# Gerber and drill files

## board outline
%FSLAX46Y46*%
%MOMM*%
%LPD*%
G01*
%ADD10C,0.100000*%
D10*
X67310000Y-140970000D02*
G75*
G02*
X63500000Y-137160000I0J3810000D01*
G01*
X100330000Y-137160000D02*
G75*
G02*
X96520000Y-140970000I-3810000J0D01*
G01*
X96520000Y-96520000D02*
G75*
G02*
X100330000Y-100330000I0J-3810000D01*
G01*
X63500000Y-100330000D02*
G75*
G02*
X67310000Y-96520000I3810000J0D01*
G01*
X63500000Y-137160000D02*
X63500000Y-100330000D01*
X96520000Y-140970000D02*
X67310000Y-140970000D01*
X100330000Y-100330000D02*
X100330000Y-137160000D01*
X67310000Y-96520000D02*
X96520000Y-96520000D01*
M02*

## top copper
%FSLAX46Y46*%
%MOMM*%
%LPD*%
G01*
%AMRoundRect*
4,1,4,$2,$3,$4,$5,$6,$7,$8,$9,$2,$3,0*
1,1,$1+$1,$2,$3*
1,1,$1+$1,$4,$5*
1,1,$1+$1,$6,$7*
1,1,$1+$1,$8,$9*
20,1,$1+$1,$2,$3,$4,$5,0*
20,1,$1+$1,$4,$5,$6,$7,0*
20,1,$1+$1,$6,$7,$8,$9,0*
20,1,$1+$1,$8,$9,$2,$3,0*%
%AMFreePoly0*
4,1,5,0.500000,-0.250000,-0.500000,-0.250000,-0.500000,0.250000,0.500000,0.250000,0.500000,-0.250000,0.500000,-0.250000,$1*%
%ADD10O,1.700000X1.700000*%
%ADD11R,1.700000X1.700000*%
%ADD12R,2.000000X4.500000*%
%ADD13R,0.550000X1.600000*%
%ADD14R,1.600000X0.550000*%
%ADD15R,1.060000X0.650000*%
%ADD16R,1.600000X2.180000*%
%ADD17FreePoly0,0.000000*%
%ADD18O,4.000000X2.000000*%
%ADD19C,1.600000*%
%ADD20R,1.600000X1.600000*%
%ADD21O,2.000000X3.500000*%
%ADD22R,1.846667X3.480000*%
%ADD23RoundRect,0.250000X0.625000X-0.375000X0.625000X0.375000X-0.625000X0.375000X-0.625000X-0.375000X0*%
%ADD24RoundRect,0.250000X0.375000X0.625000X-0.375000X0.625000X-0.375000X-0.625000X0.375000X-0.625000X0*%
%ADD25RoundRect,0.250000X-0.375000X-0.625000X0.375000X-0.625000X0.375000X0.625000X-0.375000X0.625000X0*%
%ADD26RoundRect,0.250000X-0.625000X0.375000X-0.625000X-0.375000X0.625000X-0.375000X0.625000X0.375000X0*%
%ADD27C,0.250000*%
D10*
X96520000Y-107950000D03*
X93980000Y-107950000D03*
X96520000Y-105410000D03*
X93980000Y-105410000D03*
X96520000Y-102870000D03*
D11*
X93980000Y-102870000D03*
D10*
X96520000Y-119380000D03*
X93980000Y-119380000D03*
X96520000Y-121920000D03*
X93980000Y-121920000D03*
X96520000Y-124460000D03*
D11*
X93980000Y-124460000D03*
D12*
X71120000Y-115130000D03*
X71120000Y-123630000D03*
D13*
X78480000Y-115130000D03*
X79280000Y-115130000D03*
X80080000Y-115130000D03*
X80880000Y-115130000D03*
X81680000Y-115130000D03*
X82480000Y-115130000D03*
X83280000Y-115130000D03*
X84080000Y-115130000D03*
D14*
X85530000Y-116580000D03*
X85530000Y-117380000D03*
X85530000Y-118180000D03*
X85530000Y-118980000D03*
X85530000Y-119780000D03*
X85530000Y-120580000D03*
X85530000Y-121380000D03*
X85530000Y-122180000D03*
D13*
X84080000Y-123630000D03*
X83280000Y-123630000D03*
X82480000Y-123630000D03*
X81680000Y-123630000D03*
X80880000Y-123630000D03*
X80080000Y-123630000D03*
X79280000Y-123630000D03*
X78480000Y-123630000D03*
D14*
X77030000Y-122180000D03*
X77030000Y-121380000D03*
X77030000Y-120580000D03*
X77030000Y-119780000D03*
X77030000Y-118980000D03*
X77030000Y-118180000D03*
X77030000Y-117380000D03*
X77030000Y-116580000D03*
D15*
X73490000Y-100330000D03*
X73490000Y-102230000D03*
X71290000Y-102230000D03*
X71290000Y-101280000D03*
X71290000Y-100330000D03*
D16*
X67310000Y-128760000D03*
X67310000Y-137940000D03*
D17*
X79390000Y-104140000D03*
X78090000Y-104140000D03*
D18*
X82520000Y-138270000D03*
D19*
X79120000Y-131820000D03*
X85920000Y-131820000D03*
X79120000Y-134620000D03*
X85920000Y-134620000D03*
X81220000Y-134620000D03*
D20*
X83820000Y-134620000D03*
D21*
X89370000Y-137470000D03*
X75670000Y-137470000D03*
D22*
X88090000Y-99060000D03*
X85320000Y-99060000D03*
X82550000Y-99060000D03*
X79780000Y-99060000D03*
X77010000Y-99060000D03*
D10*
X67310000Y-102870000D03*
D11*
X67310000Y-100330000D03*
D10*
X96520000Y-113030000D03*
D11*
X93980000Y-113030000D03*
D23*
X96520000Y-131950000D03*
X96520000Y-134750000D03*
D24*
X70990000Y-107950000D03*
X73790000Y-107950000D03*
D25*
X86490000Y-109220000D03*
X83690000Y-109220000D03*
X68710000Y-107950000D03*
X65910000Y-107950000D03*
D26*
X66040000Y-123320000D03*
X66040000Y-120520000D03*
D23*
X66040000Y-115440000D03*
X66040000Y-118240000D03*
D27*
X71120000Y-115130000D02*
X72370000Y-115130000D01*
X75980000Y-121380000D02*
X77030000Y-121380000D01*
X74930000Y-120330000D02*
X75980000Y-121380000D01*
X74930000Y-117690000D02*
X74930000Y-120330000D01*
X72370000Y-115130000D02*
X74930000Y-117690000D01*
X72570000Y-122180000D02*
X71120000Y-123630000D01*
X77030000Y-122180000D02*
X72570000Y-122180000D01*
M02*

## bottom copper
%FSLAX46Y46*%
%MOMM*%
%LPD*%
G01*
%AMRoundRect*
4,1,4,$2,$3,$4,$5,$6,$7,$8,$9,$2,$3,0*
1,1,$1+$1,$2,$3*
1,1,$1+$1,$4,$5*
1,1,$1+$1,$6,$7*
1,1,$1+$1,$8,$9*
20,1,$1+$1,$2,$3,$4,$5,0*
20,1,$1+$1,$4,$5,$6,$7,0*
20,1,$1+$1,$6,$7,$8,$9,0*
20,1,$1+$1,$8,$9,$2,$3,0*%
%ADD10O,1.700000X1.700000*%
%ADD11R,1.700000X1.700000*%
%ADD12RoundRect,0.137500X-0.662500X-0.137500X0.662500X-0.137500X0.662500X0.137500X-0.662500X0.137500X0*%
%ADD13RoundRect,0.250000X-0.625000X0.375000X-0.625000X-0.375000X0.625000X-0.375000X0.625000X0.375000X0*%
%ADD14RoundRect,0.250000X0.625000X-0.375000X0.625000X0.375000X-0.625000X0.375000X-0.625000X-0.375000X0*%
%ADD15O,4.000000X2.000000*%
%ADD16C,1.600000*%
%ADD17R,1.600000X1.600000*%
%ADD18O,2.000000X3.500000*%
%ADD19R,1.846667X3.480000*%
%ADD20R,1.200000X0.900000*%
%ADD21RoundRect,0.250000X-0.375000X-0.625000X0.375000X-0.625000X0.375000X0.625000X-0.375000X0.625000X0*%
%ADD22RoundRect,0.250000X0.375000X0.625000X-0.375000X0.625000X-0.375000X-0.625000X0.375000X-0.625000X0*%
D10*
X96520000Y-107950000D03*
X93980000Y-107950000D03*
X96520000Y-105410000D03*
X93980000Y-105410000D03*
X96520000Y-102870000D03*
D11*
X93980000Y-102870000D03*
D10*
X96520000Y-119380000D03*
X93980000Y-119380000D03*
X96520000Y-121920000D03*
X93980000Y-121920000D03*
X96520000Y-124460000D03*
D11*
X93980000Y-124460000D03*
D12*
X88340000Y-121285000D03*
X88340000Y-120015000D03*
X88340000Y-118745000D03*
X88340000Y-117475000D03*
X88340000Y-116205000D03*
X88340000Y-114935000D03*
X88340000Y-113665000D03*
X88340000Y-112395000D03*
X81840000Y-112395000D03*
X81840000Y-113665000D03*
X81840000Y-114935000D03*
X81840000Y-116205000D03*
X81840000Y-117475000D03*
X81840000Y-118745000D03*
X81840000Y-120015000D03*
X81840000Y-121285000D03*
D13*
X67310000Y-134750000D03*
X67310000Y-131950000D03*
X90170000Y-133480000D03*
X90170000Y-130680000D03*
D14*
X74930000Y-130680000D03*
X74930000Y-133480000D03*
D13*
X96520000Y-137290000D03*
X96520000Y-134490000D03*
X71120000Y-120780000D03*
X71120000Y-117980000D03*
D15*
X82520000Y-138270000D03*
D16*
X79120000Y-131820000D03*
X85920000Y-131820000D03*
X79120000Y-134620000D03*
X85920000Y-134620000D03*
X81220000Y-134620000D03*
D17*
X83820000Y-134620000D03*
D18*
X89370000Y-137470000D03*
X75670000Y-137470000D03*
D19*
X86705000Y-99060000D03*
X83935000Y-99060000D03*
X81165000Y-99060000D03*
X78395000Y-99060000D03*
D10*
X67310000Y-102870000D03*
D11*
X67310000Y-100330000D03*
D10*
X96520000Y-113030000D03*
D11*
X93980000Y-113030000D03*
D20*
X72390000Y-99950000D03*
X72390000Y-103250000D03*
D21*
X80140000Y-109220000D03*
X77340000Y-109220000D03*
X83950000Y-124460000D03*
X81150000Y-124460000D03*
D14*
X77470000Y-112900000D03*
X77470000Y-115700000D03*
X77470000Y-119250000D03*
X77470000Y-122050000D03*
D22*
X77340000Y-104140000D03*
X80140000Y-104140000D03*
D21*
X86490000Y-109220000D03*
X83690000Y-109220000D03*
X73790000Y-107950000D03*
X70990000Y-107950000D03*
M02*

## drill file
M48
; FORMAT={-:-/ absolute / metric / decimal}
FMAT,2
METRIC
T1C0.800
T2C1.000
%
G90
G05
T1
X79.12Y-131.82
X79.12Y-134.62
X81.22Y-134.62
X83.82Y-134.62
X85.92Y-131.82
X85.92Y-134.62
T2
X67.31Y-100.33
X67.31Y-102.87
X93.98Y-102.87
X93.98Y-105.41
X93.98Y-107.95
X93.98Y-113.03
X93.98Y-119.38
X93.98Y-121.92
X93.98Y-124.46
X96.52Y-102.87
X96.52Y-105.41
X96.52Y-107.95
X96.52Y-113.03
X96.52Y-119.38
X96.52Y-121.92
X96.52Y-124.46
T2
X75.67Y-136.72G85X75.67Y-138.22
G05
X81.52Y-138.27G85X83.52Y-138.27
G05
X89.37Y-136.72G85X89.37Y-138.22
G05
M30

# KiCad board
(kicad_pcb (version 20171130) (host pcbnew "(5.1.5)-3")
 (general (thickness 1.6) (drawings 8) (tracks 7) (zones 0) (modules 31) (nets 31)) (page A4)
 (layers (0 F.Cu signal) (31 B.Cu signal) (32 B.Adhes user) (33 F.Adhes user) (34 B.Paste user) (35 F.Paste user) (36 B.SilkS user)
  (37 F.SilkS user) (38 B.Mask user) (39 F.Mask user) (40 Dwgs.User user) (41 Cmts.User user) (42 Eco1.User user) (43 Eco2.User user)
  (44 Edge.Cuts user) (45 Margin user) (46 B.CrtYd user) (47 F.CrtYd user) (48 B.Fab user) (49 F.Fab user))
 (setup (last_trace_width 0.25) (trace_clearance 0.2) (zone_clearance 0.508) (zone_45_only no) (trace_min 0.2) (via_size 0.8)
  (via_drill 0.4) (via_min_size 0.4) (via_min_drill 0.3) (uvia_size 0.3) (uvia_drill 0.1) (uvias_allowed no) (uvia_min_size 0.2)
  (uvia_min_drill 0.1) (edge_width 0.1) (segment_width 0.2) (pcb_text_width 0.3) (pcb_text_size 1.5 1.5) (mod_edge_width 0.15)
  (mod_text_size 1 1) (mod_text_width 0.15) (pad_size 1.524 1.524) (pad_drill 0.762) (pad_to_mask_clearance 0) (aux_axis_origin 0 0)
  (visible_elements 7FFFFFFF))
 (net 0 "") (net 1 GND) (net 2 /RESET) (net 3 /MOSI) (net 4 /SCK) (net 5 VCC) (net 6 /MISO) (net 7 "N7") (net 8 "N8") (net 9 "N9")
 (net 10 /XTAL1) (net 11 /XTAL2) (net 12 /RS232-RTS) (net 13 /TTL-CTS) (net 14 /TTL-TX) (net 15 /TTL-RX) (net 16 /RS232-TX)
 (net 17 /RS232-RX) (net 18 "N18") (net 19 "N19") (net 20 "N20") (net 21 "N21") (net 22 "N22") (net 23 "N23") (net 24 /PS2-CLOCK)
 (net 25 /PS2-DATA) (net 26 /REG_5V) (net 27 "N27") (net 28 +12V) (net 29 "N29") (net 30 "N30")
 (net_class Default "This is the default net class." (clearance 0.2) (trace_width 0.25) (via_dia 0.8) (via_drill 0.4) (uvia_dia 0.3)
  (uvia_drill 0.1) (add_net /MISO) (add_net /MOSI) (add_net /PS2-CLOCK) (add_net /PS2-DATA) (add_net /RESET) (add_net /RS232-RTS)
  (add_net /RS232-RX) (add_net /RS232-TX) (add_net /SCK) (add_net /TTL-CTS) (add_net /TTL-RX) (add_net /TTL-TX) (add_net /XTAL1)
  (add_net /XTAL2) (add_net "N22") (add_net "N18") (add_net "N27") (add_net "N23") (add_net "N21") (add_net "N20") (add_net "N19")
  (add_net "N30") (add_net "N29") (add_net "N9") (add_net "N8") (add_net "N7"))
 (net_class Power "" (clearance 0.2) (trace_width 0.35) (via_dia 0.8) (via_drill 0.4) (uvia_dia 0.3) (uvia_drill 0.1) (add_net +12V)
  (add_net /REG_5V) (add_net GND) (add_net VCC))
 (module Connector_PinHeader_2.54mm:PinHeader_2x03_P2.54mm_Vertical (layer F.Cu) (at 93.98 102.87)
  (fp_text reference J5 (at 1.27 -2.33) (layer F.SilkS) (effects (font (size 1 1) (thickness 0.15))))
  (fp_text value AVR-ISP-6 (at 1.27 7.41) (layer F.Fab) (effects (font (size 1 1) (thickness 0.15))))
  (pad 6 thru_hole oval (at 2.54 5.08) (size 1.7 1.7) (drill 1) (layers *.Cu *.Mask) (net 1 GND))
  (pad 5 thru_hole oval (at 0 5.08) (size 1.7 1.7) (drill 1) (layers *.Cu *.Mask) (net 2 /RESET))
  (pad 4 thru_hole oval (at 2.54 2.54) (size 1.7 1.7) (drill 1) (layers *.Cu *.Mask) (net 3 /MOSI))
  (pad 3 thru_hole oval (at 0 2.54) (size 1.7 1.7) (drill 1) (layers *.Cu *.Mask) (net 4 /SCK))
  (pad 2 thru_hole oval (at 2.54 0) (size 1.7 1.7) (drill 1) (layers *.Cu *.Mask) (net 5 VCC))
  (pad 1 thru_hole rect (at 0 0) (size 1.7 1.7) (drill 1) (layers *.Cu *.Mask) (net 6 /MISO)))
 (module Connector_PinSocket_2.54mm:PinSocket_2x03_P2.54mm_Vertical (layer F.Cu) (at 93.98 124.46 180)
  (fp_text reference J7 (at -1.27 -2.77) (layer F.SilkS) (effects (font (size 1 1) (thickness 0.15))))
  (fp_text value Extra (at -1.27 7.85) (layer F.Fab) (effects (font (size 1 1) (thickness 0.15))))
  (pad 6 thru_hole oval (at -2.54 5.08 180) (size 1.7 1.7) (drill 1) (layers *.Cu *.Mask) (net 1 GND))
  (pad 5 thru_hole oval (at 0 5.08 180) (size 1.7 1.7) (drill 1) (layers *.Cu *.Mask) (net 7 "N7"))
  (pad 4 thru_hole oval (at -2.54 2.54 180) (size 1.7 1.7) (drill 1) (layers *.Cu *.Mask) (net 1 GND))
  (pad 3 thru_hole oval (at 0 2.54 180) (size 1.7 1.7) (drill 1) (layers *.Cu *.Mask) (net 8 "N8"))
  (pad 2 thru_hole oval (at -2.54 0 180) (size 1.7 1.7) (drill 1) (layers *.Cu *.Mask) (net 1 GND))
  (pad 1 thru_hole rect (at 0 0 180) (size 1.7 1.7) (drill 1) (layers *.Cu *.Mask) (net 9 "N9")))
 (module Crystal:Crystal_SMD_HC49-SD (layer F.Cu) (at 71.12 119.38 90)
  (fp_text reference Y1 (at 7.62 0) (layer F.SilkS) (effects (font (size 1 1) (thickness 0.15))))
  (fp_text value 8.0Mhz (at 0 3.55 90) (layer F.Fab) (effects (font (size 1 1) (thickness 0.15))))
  (pad 2 smd rect (at 4.25 0 90) (size 4.5 2) (layers F.Cu F.Paste F.Mask) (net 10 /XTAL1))
  (pad 1 smd rect (at -4.25 0 90) (size 4.5 2) (layers F.Cu F.Paste F.Mask) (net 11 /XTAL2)))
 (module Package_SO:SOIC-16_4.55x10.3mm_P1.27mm (layer B.Cu) (at 85.09 116.84)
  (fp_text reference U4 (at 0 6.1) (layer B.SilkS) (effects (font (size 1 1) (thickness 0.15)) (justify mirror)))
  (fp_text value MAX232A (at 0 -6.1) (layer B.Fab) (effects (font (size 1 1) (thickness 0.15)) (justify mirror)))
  (pad 16 smd roundrect (at 3.25 4.445) (size 1.6 0.55) (layers B.Cu B.Paste B.Mask) (roundrect_rratio 0.25) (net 5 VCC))
  (pad 15 smd roundrect (at 3.25 3.175) (size 1.6 0.55) (layers B.Cu B.Paste B.Mask) (roundrect_rratio 0.25) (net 1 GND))
  (pad 14 smd roundrect (at 3.25 1.905) (size 1.6 0.55) (layers B.Cu B.Paste B.Mask) (roundrect_rratio 0.25))
  (pad 13 smd roundrect (at 3.25 0.635) (size 1.6 0.55) (layers B.Cu B.Paste B.Mask) (roundrect_rratio 0.25) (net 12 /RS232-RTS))
  (pad 12 smd roundrect (at 3.25 -0.635) (size 1.6 0.55) (layers B.Cu B.Paste B.Mask) (roundrect_rratio 0.25) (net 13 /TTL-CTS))
  (pad 11 smd roundrect (at 3.25 -1.905) (size 1.6 0.55) (layers B.Cu B.Paste B.Mask) (roundrect_rratio 0.25) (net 1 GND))
  (pad 10 smd roundrect (at 3.25 -3.175) (size 1.6 0.55) (layers B.Cu B.Paste B.Mask) (roundrect_rratio 0.25) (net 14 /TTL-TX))
  (pad 9 smd roundrect (at 3.25 -4.445) (size 1.6 0.55) (layers B.Cu B.Paste B.Mask) (roundrect_rratio 0.25) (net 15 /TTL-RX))
  (pad 8 smd roundrect (at -3.25 -4.445) (size 1.6 0.55) (layers B.Cu B.Paste B.Mask) (roundrect_rratio 0.25) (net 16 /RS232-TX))
  (pad 7 smd roundrect (at -3.25 -3.175) (size 1.6 0.55) (layers B.Cu B.Paste B.Mask) (roundrect_rratio 0.25) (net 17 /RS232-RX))
  (pad 6 smd roundrect (at -3.25 -1.905) (size 1.6 0.55) (layers B.Cu B.Paste B.Mask) (roundrect_rratio 0.25) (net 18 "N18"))
  (pad 5 smd roundrect (at -3.25 -0.635) (size 1.6 0.55) (layers B.Cu B.Paste B.Mask) (roundrect_rratio 0.25) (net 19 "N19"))
  (pad 4 smd roundrect (at -3.25 0.635) (size 1.6 0.55) (layers B.Cu B.Paste B.Mask) (roundrect_rratio 0.25) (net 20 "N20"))
  (pad 3 smd roundrect (at -3.25 1.905) (size 1.6 0.55) (layers B.Cu B.Paste B.Mask) (roundrect_rratio 0.25) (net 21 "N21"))
  (pad 2 smd roundrect (at -3.25 3.175) (size 1.6 0.55) (layers B.Cu B.Paste B.Mask) (roundrect_rratio 0.25) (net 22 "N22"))
  (pad 1 smd roundrect (at -3.25 4.445) (size 1.6 0.55) (layers B.Cu B.Paste B.Mask) (roundrect_rratio 0.25) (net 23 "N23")))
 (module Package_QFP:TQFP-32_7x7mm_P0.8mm (layer F.Cu) (at 81.28 119.38)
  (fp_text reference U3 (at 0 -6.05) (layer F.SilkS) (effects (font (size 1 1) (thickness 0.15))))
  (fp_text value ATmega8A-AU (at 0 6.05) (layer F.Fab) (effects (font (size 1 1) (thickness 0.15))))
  (pad 32 smd rect (at -2.8 -4.25 90) (size 1.6 0.55) (layers F.Cu F.Paste F.Mask) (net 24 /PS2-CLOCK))
  (pad 31 smd rect (at -2 -4.25 90) (size 1.6 0.55) (layers F.Cu F.Paste F.Mask) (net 14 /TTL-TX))
  (pad 30 smd rect (at -1.2 -4.25 90) (size 1.6 0.55) (layers F.Cu F.Paste F.Mask) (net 15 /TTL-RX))
  (pad 29 smd rect (at -0.4 -4.25 90) (size 1.6 0.55) (layers F.Cu F.Paste F.Mask) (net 2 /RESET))
  (pad 28 smd rect (at 0.4 -4.25 90) (size 1.6 0.55) (layers F.Cu F.Paste F.Mask))
  (pad 27 smd rect (at 1.2 -4.25 90) (size 1.6 0.55) (layers F.Cu F.Paste F.Mask))
  (pad 26 smd rect (at 2 -4.25 90) (size 1.6 0.55) (layers F.Cu F.Paste F.Mask))
  (pad 25 smd rect (at 2.8 -4.25 90) (size 1.6 0.55) (layers F.Cu F.Paste F.Mask) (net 7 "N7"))
  (pad 24 smd rect (at 4.25 -2.8) (size 1.6 0.55) (layers F.Cu F.Paste F.Mask) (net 8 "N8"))
  (pad 23 smd rect (at 4.25 -2) (size 1.6 0.55) (layers F.Cu F.Paste F.Mask) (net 9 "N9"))
  (pad 22 smd rect (at 4.25 -1.2) (size 1.6 0.55) (layers F.Cu F.Paste F.Mask) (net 1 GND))
  (pad 21 smd rect (at 4.25 -0.4) (size 1.6 0.55) (layers F.Cu F.Paste F.Mask) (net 1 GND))
  (pad 20 smd rect (at 4.25 0.4) (size 1.6 0.55) (layers F.Cu F.Paste F.Mask) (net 5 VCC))
  (pad 19 smd rect (at 4.25 1.2) (size 1.6 0.55) (layers F.Cu F.Paste F.Mask) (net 1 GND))
  (pad 18 smd rect (at 4.25 2) (size 1.6 0.55) (layers F.Cu F.Paste F.Mask) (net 5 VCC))
  (pad 17 smd rect (at 4.25 2.8) (size 1.6 0.55) (layers F.Cu F.Paste F.Mask) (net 4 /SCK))
  (pad 16 smd rect (at 2.8 4.25 90) (size 1.6 0.55) (layers F.Cu F.Paste F.Mask) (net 6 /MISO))
  (pad 15 smd rect (at 2 4.25 90) (size 1.6 0.55) (layers F.Cu F.Paste F.Mask) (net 3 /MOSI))
  (pad 14 smd rect (at 1.2 4.25 90) (size 1.6 0.55) (layers F.Cu F.Paste F.Mask))
  (pad 13 smd rect (at 0.4 4.25 90) (size 1.6 0.55) (layers F.Cu F.Paste F.Mask))
  (pad 12 smd rect (at -0.4 4.25 90) (size 1.6 0.55) (layers F.Cu F.Paste F.Mask))
  (pad 11 smd rect (at -1.2 4.25 90) (size 1.6 0.55) (layers F.Cu F.Paste F.Mask))
  (pad 10 smd rect (at -2 4.25 90) (size 1.6 0.55) (layers F.Cu F.Paste F.Mask))
  (pad 9 smd rect (at -2.8 4.25 90) (size 1.6 0.55) (layers F.Cu F.Paste F.Mask))
  (pad 8 smd rect (at -4.25 2.8) (size 1.6 0.55) (layers F.Cu F.Paste F.Mask) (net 11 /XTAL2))
  (pad 7 smd rect (at -4.25 2) (size 1.6 0.55) (layers F.Cu F.Paste F.Mask) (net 10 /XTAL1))
  (pad 6 smd rect (at -4.25 1.2) (size 1.6 0.55) (layers F.Cu F.Paste F.Mask) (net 5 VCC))
  (pad 5 smd rect (at -4.25 0.4) (size 1.6 0.55) (layers F.Cu F.Paste F.Mask) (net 1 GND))
  (pad 4 smd rect (at -4.25 -0.4) (size 1.6 0.55) (layers F.Cu F.Paste F.Mask) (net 5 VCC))
  (pad 3 smd rect (at -4.25 -1.2) (size 1.6 0.55) (layers F.Cu F.Paste F.Mask) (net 1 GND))
  (pad 2 smd rect (at -4.25 -2) (size 1.6 0.55) (layers F.Cu F.Paste F.Mask) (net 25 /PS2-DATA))
  (pad 1 smd rect (at -4.25 -2.8) (size 1.6 0.55) (layers F.Cu F.Paste F.Mask) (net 13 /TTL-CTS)))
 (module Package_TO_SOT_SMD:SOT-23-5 (layer F.Cu) (at 72.39 101.28)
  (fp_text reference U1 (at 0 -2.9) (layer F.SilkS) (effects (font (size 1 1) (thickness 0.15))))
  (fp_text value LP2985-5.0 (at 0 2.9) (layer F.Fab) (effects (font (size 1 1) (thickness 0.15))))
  (pad 5 smd rect (at 1.1 -0.95) (size 1.06 0.65) (layers F.Cu F.Paste F.Mask) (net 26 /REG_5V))
  (pad 4 smd rect (at 1.1 0.95) (size 1.06 0.65) (layers F.Cu F.Paste F.Mask) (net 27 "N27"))
  (pad 3 smd rect (at -1.1 0.95) (size 1.06 0.65) (layers F.Cu F.Paste F.Mask) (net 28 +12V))
  (pad 2 smd rect (at -1.1 0) (size 1.06 0.65) (layers F.Cu F.Paste F.Mask) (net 1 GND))
  (pad 1 smd rect (at -1.1 -0.95) (size 1.06 0.65) (layers F.Cu F.Paste F.Mask) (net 28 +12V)))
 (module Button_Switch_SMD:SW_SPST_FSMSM (layer F.Cu) (at 67.31 133.35 90)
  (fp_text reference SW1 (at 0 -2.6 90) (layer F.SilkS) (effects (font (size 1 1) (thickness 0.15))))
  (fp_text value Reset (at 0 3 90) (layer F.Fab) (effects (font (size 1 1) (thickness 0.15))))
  (pad 2 smd rect (at 4.59 0 90) (size 2.18 1.6) (layers F.Cu F.Paste F.Mask) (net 1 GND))
  (pad 1 smd rect (at -4.59 0 90) (size 2.18 1.6) (layers F.Cu F.Paste F.Mask) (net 2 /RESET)))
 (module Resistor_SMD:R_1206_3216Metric (layer B.Cu) (at 67.31 133.35 270)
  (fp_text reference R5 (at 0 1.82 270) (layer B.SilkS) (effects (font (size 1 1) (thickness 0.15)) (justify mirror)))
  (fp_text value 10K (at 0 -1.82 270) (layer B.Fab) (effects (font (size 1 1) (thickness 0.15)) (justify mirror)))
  (pad 2 smd roundrect (at 1.4 0 270) (size 1.25 1.75) (layers B.Cu B.Paste B.Mask) (roundrect_rratio 0.2) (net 2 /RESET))
  (pad 1 smd roundrect (at -1.4 0 270) (size 1.25 1.75) (layers B.Cu B.Paste B.Mask) (roundrect_rratio 0.2) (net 5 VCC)))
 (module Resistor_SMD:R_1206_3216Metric (layer B.Cu) (at 90.17 132.08 270)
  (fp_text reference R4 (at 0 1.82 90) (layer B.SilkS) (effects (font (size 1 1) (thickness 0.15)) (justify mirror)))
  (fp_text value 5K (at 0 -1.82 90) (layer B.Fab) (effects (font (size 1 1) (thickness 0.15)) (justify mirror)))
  (pad 2 smd roundrect (at 1.4 0 270) (size 1.25 1.75) (layers B.Cu B.Paste B.Mask) (roundrect_rratio 0.2) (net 24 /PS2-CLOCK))
  (pad 1 smd roundrect (at -1.4 0 270) (size 1.25 1.75) (layers B.Cu B.Paste B.Mask) (roundrect_rratio 0.2) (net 5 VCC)))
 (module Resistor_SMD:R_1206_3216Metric (layer B.Cu) (at 74.93 132.08 90)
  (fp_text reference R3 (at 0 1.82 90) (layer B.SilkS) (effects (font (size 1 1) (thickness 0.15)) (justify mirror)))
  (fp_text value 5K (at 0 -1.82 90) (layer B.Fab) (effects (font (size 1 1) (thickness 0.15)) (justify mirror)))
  (pad 2 smd roundrect (at 1.4 0 90) (size 1.25 1.75) (layers B.Cu B.Paste B.Mask) (roundrect_rratio 0.2) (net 25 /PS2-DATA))
  (pad 1 smd roundrect (at -1.4 0 90) (size 1.25 1.75) (layers B.Cu B.Paste B.Mask) (roundrect_rratio 0.2) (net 5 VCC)))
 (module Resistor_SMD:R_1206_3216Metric (layer B.Cu) (at 96.52 135.89 270)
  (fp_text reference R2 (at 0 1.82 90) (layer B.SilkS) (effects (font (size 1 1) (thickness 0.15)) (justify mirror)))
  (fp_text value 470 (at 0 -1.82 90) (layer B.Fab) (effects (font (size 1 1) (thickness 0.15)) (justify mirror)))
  (pad 2 smd roundrect (at 1.4 0 270) (size 1.25 1.75) (layers B.Cu B.Paste B.Mask) (roundrect_rratio 0.2) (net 1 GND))
  (pad 1 smd roundrect (at -1.4 0 270) (size 1.25 1.75) (layers B.Cu B.Paste B.Mask) (roundrect_rratio 0.2) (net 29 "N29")))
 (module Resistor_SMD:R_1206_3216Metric (layer B.Cu) (at 71.12 119.38 270)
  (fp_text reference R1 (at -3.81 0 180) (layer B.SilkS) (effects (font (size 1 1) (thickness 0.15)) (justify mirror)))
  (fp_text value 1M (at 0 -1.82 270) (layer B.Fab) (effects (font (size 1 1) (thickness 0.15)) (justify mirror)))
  (pad 2 smd roundrect (at 1.4 0 270) (size 1.25 1.75) (layers B.Cu B.Paste B.Mask) (roundrect_rratio 0.2) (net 11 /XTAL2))
  (pad 1 smd roundrect (at -1.4 0 270) (size 1.25 1.75) (layers B.Cu B.Paste B.Mask) (roundrect_rratio 0.2) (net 10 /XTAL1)))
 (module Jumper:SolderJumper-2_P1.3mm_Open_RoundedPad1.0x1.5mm (layer F.Cu) (at 78.74 104.14)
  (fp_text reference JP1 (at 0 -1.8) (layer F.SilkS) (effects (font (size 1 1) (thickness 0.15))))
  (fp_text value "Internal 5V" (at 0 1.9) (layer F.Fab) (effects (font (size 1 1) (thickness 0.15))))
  (pad 2 smd custom (at 0.65 0) (size 1 0.5) (layers F.Cu F.Mask) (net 5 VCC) (zone_connect 2) (options (clearance outline) (anchor rect))
   (primitives))
  (pad 1 smd custom (at -0.65 0) (size 1 0.5) (layers F.Cu F.Mask) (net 26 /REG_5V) (zone_connect 2)
   (options (clearance outline) (anchor rect)) (primitives)))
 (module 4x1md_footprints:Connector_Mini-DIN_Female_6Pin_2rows (layer F.Cu) (at 83.82 134.62)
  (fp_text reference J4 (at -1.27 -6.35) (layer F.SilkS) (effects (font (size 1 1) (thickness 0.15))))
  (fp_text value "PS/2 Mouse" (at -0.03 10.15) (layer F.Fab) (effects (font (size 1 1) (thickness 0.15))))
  (pad 7 thru_hole oval (at -1.3 3.65) (size 4 2) (drill oval 3 1) (layers *.Cu *.Mask) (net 1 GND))
  (pad 6 thru_hole circle (at -4.7 -2.8) (size 1.6 1.6) (drill 0.8) (layers *.Cu *.Mask))
  (pad 5 thru_hole circle (at 2.1 -2.8) (size 1.6 1.6) (drill 0.8) (layers *.Cu *.Mask) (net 24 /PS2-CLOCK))
  (pad 4 thru_hole circle (at -4.7 0) (size 1.6 1.6) (drill 0.8) (layers *.Cu *.Mask) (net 5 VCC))
  (pad 3 thru_hole circle (at 2.1 0) (size 1.6 1.6) (drill 0.8) (layers *.Cu *.Mask) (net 1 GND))
  (pad 2 thru_hole circle (at -2.6 0) (size 1.6 1.6) (drill 0.8) (layers *.Cu *.Mask))
  (pad 1 thru_hole rect (at 0 0) (size 1.6 1.6) (drill 0.8) (layers *.Cu *.Mask) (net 25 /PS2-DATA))
  (pad 7 thru_hole oval (at 5.55 2.85) (size 2 3.5) (drill oval 1 2.5) (layers *.Cu *.Mask) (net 1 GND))
  (pad 7 thru_hole oval (at -8.15 2.85) (size 2 3.5) (drill oval 1 2.5) (layers *.Cu *.Mask) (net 1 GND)))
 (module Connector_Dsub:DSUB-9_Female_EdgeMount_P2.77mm (layer F.Cu) (at 82.55 99.06 180)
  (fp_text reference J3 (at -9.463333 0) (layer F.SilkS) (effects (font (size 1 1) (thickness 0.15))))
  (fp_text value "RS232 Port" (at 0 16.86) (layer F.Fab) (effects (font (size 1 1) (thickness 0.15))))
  (pad 9 smd rect (at -4.155 0 180) (size 1.846667 3.48) (layers B.Cu B.Paste B.Mask))
  (pad 8 smd rect (at -1.385 0 180) (size 1.846667 3.48) (layers B.Cu B.Paste B.Mask))
  (pad 7 smd rect (at 1.385 0 180) (size 1.846667 3.48) (layers B.Cu B.Paste B.Mask) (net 12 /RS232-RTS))
  (pad 6 smd rect (at 4.155 0 180) (size 1.846667 3.48) (layers B.Cu B.Paste B.Mask))
  (pad 5 smd rect (at -5.54 0 180) (size 1.846667 3.48) (layers F.Cu F.Paste F.Mask) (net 1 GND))
  (pad 4 smd rect (at -2.77 0 180) (size 1.846667 3.48) (layers F.Cu F.Paste F.Mask))
  (pad 3 smd rect (at 0 0 180) (size 1.846667 3.48) (layers F.Cu F.Paste F.Mask) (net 16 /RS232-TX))
  (pad 2 smd rect (at 2.77 0 180) (size 1.846667 3.48) (layers F.Cu F.Paste F.Mask) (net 17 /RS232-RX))
  (pad 1 smd rect (at 5.54 0 180) (size 1.846667 3.48) (layers F.Cu F.Paste F.Mask)))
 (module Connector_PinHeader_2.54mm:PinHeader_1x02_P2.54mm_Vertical (layer F.Cu) (at 67.31 100.33)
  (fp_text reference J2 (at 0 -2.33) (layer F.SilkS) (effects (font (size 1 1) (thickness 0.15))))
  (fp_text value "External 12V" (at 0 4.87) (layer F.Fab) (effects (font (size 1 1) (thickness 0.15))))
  (pad 2 thru_hole oval (at 0 2.54) (size 1.7 1.7) (drill 1) (layers *.Cu *.Mask) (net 1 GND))
  (pad 1 thru_hole rect (at 0 0) (size 1.7 1.7) (drill 1) (layers *.Cu *.Mask) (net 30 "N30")))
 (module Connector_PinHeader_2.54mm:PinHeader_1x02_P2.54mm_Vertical (layer F.Cu) (at 93.98 113.03 90)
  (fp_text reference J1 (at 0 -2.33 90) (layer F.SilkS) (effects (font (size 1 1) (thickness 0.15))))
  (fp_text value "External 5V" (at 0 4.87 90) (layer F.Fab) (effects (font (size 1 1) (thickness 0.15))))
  (pad 2 thru_hole oval (at 0 2.54 90) (size 1.7 1.7) (drill 1) (layers *.Cu *.Mask) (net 1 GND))
  (pad 1 thru_hole rect (at 0 0 90) (size 1.7 1.7) (drill 1) (layers *.Cu *.Mask) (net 5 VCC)))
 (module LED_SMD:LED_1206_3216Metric (layer F.Cu) (at 96.52 133.35 90)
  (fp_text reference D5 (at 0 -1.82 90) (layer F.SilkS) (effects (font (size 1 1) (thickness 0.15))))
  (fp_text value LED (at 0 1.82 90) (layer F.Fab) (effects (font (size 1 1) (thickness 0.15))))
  (pad 2 smd roundrect (at 1.4 0 90) (size 1.25 1.75) (layers F.Cu F.Paste F.Mask) (roundrect_rratio 0.2) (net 4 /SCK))
  (pad 1 smd roundrect (at -1.4 0 90) (size 1.25 1.75) (layers F.Cu F.Paste F.Mask) (roundrect_rratio 0.2) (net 29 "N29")))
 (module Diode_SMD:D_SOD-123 (layer B.Cu) (at 72.39 101.6 90)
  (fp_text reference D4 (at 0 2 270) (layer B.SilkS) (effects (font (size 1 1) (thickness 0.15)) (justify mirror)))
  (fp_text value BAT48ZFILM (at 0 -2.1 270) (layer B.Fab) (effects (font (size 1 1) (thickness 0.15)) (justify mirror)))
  (pad 2 smd rect (at 1.65 0 90) (size 0.9 1.2) (layers B.Cu B.Paste B.Mask) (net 30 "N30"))
  (pad 1 smd rect (at -1.65 0 90) (size 0.9 1.2) (layers B.Cu B.Paste B.Mask) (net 28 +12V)))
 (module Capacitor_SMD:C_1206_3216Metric (layer F.Cu) (at 72.39 107.95 180)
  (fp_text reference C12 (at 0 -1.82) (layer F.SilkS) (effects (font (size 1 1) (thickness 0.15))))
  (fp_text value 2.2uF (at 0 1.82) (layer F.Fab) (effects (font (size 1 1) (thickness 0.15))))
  (pad 2 smd roundrect (at 1.4 0 180) (size 1.25 1.75) (layers F.Cu F.Paste F.Mask) (roundrect_rratio 0.2) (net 1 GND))
  (pad 1 smd roundrect (at -1.4 0 180) (size 1.25 1.75) (layers F.Cu F.Paste F.Mask) (roundrect_rratio 0.2) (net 26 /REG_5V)))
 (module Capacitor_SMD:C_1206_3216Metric (layer B.Cu) (at 78.74 109.22)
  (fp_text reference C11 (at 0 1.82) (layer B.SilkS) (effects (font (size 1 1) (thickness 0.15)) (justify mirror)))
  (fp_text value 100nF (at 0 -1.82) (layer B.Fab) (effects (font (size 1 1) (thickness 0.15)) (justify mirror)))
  (pad 2 smd roundrect (at 1.4 0) (size 1.25 1.75) (layers B.Cu B.Paste B.Mask) (roundrect_rratio 0.2) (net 1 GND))
  (pad 1 smd roundrect (at -1.4 0) (size 1.25 1.75) (layers B.Cu B.Paste B.Mask) (roundrect_rratio 0.2) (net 18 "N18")))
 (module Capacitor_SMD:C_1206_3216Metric (layer B.Cu) (at 82.55 124.46)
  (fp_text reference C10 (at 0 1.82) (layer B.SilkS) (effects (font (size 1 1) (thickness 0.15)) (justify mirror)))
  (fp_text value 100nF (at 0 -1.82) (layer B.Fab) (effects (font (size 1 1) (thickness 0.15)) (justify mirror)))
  (pad 2 smd roundrect (at 1.4 0) (size 1.25 1.75) (layers B.Cu B.Paste B.Mask) (roundrect_rratio 0.2) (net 5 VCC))
  (pad 1 smd roundrect (at -1.4 0) (size 1.25 1.75) (layers B.Cu B.Paste B.Mask) (roundrect_rratio 0.2) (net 22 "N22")))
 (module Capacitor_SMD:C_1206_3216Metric (layer B.Cu) (at 77.47 114.3 90)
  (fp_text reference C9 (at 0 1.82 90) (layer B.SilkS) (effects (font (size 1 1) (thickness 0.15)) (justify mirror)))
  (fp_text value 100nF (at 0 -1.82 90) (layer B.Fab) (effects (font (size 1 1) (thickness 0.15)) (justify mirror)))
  (pad 2 smd roundrect (at 1.4 0 90) (size 1.25 1.75) (layers B.Cu B.Paste B.Mask) (roundrect_rratio 0.2) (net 19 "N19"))
  (pad 1 smd roundrect (at -1.4 0 90) (size 1.25 1.75) (layers B.Cu B.Paste B.Mask) (roundrect_rratio 0.2) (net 20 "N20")))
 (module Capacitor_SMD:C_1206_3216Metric (layer B.Cu) (at 77.47 120.65 90)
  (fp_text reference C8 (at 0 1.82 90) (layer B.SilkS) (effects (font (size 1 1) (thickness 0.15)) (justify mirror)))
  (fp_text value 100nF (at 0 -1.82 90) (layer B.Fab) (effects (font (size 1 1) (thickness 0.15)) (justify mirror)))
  (pad 2 smd roundrect (at 1.4 0 90) (size 1.25 1.75) (layers B.Cu B.Paste B.Mask) (roundrect_rratio 0.2) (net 21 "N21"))
  (pad 1 smd roundrect (at -1.4 0 90) (size 1.25 1.75) (layers B.Cu B.Paste B.Mask) (roundrect_rratio 0.2) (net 23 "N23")))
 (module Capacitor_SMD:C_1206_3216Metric (layer B.Cu) (at 78.74 104.14 180)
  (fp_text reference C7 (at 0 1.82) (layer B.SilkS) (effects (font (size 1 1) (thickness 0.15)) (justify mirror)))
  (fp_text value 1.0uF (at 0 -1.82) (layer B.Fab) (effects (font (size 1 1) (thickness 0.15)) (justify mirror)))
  (pad 2 smd roundrect (at 1.4 0 180) (size 1.25 1.75) (layers B.Cu B.Paste B.Mask) (roundrect_rratio 0.2) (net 1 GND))
  (pad 1 smd roundrect (at -1.4 0 180) (size 1.25 1.75) (layers B.Cu B.Paste B.Mask) (roundrect_rratio 0.2) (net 5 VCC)))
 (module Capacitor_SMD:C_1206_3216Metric (layer B.Cu) (at 85.09 109.22)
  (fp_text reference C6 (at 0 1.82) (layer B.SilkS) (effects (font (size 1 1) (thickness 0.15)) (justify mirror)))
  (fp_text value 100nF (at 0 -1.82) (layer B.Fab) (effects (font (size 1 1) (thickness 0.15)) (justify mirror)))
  (pad 2 smd roundrect (at 1.4 0) (size 1.25 1.75) (layers B.Cu B.Paste B.Mask) (roundrect_rratio 0.2) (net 1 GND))
  (pad 1 smd roundrect (at -1.4 0) (size 1.25 1.75) (layers B.Cu B.Paste B.Mask) (roundrect_rratio 0.2) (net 5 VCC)))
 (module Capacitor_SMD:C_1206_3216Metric (layer F.Cu) (at 85.09 109.22)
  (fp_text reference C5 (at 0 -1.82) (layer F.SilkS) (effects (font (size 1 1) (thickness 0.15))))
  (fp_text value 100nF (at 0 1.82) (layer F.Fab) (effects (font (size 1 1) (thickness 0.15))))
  (pad 2 smd roundrect (at 1.4 0) (size 1.25 1.75) (layers F.Cu F.Paste F.Mask) (roundrect_rratio 0.2) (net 1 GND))
  (pad 1 smd roundrect (at -1.4 0) (size 1.25 1.75) (layers F.Cu F.Paste F.Mask) (roundrect_rratio 0.2) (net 5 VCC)))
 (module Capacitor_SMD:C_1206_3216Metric (layer F.Cu) (at 67.31 107.95)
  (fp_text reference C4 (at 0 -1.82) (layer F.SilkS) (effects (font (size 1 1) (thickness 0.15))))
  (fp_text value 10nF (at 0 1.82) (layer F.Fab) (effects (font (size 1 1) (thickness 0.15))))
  (pad 2 smd roundrect (at 1.4 0) (size 1.25 1.75) (layers F.Cu F.Paste F.Mask) (roundrect_rratio 0.2) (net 1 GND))
  (pad 1 smd roundrect (at -1.4 0) (size 1.25 1.75) (layers F.Cu F.Paste F.Mask) (roundrect_rratio 0.2) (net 27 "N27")))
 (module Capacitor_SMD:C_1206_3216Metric (layer B.Cu) (at 72.39 107.95)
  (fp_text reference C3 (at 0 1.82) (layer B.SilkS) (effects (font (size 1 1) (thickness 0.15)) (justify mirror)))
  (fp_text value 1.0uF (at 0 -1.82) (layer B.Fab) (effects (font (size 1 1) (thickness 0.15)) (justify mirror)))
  (pad 2 smd roundrect (at 1.4 0) (size 1.25 1.75) (layers B.Cu B.Paste B.Mask) (roundrect_rratio 0.2) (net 1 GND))
  (pad 1 smd roundrect (at -1.4 0) (size 1.25 1.75) (layers B.Cu B.Paste B.Mask) (roundrect_rratio 0.2) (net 28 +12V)))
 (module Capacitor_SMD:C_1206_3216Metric (layer F.Cu) (at 66.04 121.92 270)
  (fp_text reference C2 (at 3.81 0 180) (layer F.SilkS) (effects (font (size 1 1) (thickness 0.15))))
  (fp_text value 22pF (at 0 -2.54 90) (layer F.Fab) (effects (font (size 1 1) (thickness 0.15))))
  (pad 2 smd roundrect (at 1.4 0 270) (size 1.25 1.75) (layers F.Cu F.Paste F.Mask) (roundrect_rratio 0.2) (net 11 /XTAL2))
  (pad 1 smd roundrect (at -1.4 0 270) (size 1.25 1.75) (layers F.Cu F.Paste F.Mask) (roundrect_rratio 0.2) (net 1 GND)))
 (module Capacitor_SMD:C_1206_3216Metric (layer F.Cu) (at 66.04 116.84 90)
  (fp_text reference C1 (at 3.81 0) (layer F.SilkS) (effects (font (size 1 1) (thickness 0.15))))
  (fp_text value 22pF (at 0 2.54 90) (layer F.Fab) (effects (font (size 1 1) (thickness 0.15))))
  (pad 2 smd roundrect (at 1.4 0 90) (size 1.25 1.75) (layers F.Cu F.Paste F.Mask) (roundrect_rratio 0.2) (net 10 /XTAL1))
  (pad 1 smd roundrect (at -1.4 0 90) (size 1.25 1.75) (layers F.Cu F.Paste F.Mask) (roundrect_rratio 0.2) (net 1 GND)))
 (gr_arc (start 67.31 137.16) (end 63.5 137.16) (angle -90) (layer Edge.Cuts) (width 0.1))
 (gr_arc (start 96.52 137.16) (end 96.52 140.97) (angle -90) (layer Edge.Cuts) (width 0.1))
 (gr_arc (start 96.52 100.33) (end 100.33 100.33) (angle -90) (layer Edge.Cuts) (width 0.1))
 (gr_arc (start 67.31 100.33) (end 67.31 96.52) (angle -90) (layer Edge.Cuts) (width 0.1))
 (gr_line (start 63.5 137.16) (end 63.5 100.33) (layer Edge.Cuts) (width 0.1))
 (gr_line (start 96.52 140.97) (end 67.31 140.97) (layer Edge.Cuts) (width 0.1))
 (gr_line (start 100.33 100.33) (end 100.33 137.16) (layer Edge.Cuts) (width 0.1))
 (gr_line (start 67.31 96.52) (end 96.52 96.52) (layer Edge.Cuts) (width 0.1))
 (segment (start 71.12 115.13) (end 72.37 115.13) (width 0.25) (layer F.Cu) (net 10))
 (segment (start 75.98 121.38) (end 77.03 121.38) (width 0.25) (layer F.Cu) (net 10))
 (segment (start 74.93 120.33) (end 75.98 121.38) (width 0.25) (layer F.Cu) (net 10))
 (segment (start 74.93 117.69) (end 74.93 120.33) (width 0.25) (layer F.Cu) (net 10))
 (segment (start 72.37 115.13) (end 74.93 117.69) (width 0.25) (layer F.Cu) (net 10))
 (segment (start 72.57 122.18) (end 71.12 123.63) (width 0.25) (layer F.Cu) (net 11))
 (segment (start 77.03 122.18) (end 72.57 122.18) (width 0.25) (layer F.Cu) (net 11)))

